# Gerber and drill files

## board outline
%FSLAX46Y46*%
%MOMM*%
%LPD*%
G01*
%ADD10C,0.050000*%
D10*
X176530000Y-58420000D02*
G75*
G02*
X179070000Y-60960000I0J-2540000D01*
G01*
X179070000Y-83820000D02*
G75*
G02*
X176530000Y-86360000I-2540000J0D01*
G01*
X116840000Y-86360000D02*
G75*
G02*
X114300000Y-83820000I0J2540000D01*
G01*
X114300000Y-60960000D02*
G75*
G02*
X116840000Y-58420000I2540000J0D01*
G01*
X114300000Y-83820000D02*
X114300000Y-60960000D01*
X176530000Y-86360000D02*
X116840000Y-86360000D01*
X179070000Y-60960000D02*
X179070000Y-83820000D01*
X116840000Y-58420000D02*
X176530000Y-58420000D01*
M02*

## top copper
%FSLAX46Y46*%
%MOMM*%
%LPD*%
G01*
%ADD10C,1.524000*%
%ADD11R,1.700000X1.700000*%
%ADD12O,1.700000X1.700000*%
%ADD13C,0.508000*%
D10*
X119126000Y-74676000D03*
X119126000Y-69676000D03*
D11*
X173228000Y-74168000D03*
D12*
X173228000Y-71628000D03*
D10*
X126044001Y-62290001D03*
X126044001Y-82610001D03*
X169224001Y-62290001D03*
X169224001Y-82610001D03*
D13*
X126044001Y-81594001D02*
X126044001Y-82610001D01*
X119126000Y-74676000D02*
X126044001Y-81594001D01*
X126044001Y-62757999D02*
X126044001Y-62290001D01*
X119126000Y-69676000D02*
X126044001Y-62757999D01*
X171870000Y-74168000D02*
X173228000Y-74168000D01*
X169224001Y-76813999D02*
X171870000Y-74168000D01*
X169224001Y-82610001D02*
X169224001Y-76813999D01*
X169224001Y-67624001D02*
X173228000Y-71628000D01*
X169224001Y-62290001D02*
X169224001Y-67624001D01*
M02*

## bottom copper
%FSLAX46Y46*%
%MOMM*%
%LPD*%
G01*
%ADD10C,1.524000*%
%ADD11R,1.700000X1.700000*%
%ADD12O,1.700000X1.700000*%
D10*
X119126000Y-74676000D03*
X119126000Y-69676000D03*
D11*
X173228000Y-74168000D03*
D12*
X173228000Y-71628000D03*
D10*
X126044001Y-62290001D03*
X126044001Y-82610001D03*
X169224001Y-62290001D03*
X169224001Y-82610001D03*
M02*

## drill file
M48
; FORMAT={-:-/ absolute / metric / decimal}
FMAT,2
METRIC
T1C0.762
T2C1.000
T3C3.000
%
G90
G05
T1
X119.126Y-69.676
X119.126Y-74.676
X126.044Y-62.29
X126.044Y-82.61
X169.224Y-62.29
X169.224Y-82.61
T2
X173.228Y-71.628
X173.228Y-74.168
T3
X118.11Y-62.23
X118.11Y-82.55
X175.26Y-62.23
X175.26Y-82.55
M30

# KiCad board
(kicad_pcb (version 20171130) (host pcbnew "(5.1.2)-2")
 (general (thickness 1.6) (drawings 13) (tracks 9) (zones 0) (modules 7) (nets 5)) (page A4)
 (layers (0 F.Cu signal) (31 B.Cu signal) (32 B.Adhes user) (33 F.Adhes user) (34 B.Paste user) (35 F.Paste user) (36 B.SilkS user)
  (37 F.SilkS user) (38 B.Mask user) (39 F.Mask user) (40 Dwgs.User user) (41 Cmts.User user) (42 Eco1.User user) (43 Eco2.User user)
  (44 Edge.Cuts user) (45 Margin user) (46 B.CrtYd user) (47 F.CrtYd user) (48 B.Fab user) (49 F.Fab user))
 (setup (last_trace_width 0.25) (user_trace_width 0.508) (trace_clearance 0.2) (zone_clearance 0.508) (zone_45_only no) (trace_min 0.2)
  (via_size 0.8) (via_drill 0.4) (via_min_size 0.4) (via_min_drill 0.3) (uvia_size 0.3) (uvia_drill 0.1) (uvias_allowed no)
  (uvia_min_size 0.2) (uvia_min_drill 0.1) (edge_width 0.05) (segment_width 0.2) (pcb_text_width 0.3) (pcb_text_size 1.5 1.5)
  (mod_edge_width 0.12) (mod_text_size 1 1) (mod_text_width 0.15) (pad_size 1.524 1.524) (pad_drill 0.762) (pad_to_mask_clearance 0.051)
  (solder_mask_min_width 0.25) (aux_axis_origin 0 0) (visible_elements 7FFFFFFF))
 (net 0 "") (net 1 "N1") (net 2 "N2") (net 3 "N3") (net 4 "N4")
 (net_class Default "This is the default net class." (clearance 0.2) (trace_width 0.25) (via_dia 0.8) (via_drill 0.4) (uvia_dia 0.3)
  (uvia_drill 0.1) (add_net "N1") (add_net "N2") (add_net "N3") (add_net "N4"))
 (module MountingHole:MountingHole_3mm (layer F.Cu) (at 175.26 62.23)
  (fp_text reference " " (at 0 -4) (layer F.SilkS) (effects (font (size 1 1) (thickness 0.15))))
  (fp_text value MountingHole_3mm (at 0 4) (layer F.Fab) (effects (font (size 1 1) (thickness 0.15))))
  (pad 1 np_thru_hole circle (at 0 0) (size 3 3) (drill 3) (layers *.Cu *.Mask)))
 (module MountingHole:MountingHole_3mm (layer F.Cu) (at 175.26 82.55)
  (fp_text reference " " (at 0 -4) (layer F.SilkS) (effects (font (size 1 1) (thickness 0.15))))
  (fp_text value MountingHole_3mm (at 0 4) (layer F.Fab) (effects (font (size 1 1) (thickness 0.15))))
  (pad 1 np_thru_hole circle (at 0 0) (size 3 3) (drill 3) (layers *.Cu *.Mask)))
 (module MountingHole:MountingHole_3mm (layer F.Cu) (at 118.11 82.55)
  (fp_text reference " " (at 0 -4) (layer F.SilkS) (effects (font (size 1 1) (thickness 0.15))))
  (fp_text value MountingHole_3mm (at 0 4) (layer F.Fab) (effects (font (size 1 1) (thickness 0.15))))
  (pad 1 np_thru_hole circle (at 0 0) (size 3 3) (drill 3) (layers *.Cu *.Mask)))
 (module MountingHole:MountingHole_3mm (layer F.Cu) (at 118.11 62.23)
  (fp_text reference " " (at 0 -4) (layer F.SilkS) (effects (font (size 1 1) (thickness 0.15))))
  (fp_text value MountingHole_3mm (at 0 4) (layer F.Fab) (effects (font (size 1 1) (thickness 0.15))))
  (pad 1 np_thru_hole circle (at 0 0) (size 3 3) (drill 3) (layers *.Cu *.Mask)))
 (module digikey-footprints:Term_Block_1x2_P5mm (layer F.Cu) (at 119.126 74.676 90)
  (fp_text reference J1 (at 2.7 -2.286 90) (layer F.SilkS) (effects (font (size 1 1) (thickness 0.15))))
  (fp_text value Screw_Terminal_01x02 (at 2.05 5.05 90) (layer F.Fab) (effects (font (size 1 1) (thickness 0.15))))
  (pad 1 thru_hole circle (at 0 0 90) (size 1.524 1.524) (drill 0.762) (layers *.Cu *.Mask) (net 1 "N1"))
  (pad 2 thru_hole circle (at 5 0 90) (size 1.524 1.524) (drill 0.762) (layers *.Cu *.Mask) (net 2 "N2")))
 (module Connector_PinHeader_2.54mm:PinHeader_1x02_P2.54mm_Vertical (layer F.Cu) (at 173.228 74.168 180)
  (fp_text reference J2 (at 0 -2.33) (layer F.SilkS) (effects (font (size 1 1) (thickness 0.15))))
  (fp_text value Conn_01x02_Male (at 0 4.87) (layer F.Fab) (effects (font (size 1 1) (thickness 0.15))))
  (pad 1 thru_hole rect (at 0 0 180) (size 1.7 1.7) (drill 1) (layers *.Cu *.Mask) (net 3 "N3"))
  (pad 2 thru_hole oval (at 0 2.54 180) (size 1.7 1.7) (drill 1) (layers *.Cu *.Mask) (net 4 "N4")))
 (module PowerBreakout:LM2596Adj (layer F.Cu) (at 148.904001 72.450001)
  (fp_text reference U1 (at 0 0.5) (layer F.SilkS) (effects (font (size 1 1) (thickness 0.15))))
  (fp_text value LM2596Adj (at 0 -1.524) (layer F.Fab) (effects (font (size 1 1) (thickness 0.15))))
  (pad 1 thru_hole circle (at -22.86 -10.16) (size 1.524 1.524) (drill 0.762) (layers *.Cu *.Mask) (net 2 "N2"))
  (pad 2 thru_hole circle (at -22.86 10.16) (size 1.524 1.524) (drill 0.762) (layers *.Cu *.Mask) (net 1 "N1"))
  (pad 3 thru_hole circle (at 20.32 -10.16) (size 1.524 1.524) (drill 0.762) (layers *.Cu *.Mask) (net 4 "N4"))
  (pad 4 thru_hole circle (at 20.32 10.16) (size 1.524 1.524) (drill 0.762) (layers *.Cu *.Mask) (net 3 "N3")))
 (gr_arc (start 176.53 60.96) (end 179.07 60.96) (angle -90) (layer Edge.Cuts) (width 0.05))
 (gr_arc (start 176.53 83.82) (end 176.53 86.36) (angle -90) (layer Edge.Cuts) (width 0.05))
 (gr_arc (start 116.84 83.82) (end 114.3 83.82) (angle -90) (layer Edge.Cuts) (width 0.05))
 (gr_arc (start 116.84 60.96) (end 116.84 58.42) (angle -90) (layer Edge.Cuts) (width 0.05))
 (gr_line (start 114.3 83.82) (end 114.3 60.96) (layer Edge.Cuts) (width 0.05))
 (gr_line (start 176.53 86.36) (end 116.84 86.36) (layer Edge.Cuts) (width 0.05))
 (gr_line (start 179.07 60.96) (end 179.07 83.82) (layer Edge.Cuts) (width 0.05))
 (gr_line (start 116.84 58.42) (end 176.53 58.42) (layer Edge.Cuts) (width 0.05))
 (segment (start 126.044001 81.594001) (end 126.044001 82.610001) (width 0.508) (layer F.Cu) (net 1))
 (segment (start 119.126 74.676) (end 126.044001 81.594001) (width 0.508) (layer F.Cu) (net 1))
 (segment (start 126.044001 62.757999) (end 126.044001 62.290001) (width 0.508) (layer F.Cu) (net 2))
 (segment (start 119.126 69.676) (end 126.044001 62.757999) (width 0.508) (layer F.Cu) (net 2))
 (segment (start 171.87 74.168) (end 173.228 74.168) (width 0.508) (layer F.Cu) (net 3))
 (segment (start 169.224001 76.813999) (end 171.87 74.168) (width 0.508) (layer F.Cu) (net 3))
 (segment (start 169.224001 82.610001) (end 169.224001 76.813999) (width 0.508) (layer F.Cu) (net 3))
 (segment (start 169.224001 67.624001) (end 173.228 71.628) (width 0.508) (layer F.Cu) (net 4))
 (segment (start 169.224001 62.290001) (end 169.224001 67.624001) (width 0.508) (layer F.Cu) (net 4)))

